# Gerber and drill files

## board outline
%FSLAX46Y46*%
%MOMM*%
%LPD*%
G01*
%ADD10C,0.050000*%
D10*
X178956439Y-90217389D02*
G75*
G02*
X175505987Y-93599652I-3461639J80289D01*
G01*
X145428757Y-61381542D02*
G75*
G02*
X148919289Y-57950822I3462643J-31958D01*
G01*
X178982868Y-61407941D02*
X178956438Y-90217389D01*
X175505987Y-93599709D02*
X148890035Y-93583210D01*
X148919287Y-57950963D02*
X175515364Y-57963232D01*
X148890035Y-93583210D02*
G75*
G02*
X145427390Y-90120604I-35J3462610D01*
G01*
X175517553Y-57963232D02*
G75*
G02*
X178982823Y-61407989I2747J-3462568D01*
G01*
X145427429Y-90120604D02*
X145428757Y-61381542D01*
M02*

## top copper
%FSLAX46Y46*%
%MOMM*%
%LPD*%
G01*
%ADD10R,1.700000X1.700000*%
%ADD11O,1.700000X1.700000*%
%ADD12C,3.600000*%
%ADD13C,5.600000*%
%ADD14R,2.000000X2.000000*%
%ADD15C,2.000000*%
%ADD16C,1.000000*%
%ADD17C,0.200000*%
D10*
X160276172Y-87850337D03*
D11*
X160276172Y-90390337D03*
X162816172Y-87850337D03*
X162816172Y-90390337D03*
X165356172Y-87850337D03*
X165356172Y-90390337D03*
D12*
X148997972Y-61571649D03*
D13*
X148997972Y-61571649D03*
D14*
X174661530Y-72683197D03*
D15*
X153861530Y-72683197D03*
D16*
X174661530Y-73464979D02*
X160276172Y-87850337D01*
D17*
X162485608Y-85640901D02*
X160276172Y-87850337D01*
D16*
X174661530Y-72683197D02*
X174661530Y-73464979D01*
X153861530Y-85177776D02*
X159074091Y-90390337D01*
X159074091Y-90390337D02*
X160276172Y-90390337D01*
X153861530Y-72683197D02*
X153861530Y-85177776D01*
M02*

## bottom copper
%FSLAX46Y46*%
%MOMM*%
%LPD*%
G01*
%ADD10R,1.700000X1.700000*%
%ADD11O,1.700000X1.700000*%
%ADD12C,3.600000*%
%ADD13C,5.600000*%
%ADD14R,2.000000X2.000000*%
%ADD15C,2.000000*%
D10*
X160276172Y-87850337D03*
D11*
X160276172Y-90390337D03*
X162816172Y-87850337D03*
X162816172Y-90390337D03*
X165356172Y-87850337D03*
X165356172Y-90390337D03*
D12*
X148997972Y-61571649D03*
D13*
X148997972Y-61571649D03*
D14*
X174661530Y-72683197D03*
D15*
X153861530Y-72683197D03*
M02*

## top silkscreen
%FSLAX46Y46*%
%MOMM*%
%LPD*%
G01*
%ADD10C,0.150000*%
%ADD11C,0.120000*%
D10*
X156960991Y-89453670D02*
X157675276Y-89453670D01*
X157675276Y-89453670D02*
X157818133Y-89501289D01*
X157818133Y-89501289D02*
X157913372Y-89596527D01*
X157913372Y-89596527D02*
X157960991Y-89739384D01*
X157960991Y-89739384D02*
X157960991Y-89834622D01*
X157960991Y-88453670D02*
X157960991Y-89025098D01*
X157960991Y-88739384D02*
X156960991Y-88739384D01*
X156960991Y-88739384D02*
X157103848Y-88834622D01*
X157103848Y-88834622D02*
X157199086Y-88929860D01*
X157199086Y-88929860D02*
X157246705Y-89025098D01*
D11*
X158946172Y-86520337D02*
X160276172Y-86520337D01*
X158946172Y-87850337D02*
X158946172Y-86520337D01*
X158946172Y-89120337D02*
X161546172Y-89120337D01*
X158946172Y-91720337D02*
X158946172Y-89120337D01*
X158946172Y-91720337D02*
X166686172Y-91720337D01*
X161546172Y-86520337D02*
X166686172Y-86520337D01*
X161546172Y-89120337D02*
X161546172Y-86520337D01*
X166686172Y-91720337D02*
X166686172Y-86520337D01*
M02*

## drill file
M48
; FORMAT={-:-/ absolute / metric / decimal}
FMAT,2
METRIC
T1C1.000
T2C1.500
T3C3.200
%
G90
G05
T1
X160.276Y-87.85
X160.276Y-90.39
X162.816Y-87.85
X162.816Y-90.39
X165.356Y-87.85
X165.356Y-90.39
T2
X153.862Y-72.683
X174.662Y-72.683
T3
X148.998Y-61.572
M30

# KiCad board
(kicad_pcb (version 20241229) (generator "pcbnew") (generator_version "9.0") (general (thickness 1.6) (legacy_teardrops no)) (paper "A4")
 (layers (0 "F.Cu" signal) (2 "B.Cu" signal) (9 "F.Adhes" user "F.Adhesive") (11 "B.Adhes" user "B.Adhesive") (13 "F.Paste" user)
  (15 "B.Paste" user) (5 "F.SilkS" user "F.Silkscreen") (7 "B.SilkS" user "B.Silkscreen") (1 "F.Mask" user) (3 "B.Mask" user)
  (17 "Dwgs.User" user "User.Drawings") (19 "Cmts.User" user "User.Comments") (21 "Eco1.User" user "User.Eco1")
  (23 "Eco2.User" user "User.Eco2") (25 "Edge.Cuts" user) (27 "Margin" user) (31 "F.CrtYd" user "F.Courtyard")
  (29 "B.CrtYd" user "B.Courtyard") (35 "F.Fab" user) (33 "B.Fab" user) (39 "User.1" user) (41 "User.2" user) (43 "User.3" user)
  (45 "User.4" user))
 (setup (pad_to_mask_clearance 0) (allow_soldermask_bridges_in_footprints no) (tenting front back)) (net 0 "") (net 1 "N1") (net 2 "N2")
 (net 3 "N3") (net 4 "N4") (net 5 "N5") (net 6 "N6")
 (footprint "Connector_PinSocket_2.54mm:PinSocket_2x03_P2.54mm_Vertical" (layer "F.Cu") (at 160.276172 87.850337 90)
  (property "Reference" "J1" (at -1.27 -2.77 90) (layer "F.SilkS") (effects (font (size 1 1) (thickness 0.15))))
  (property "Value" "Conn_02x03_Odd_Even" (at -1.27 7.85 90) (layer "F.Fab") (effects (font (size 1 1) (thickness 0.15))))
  (fp_line (start 1.33 -1.33) (end 1.33 0) (stroke (width 0.12) (type solid)) (layer "F.SilkS"))
  (fp_line (start 0 -1.33) (end 1.33 -1.33) (stroke (width 0.12) (type solid)) (layer "F.SilkS"))
  (fp_line (start -1.27 -1.33) (end -1.27 1.27) (stroke (width 0.12) (type solid)) (layer "F.SilkS"))
  (fp_line (start -3.87 -1.33) (end -1.27 -1.33) (stroke (width 0.12) (type solid)) (layer "F.SilkS"))
  (fp_line (start -3.87 -1.33) (end -3.87 6.41) (stroke (width 0.12) (type solid)) (layer "F.SilkS"))
  (fp_line (start 1.33 1.27) (end 1.33 6.41) (stroke (width 0.12) (type solid)) (layer "F.SilkS"))
  (fp_line (start -1.27 1.27) (end 1.33 1.27) (stroke (width 0.12) (type solid)) (layer "F.SilkS"))
  (fp_line (start -3.87 6.41) (end 1.33 6.41) (stroke (width 0.12) (type solid)) (layer "F.SilkS"))
  (pad "1" thru_hole rect (at 0 0 90) (size 1.7 1.7) (drill 1) (layers "*.Cu" "*.Mask") (remove_unused_layers no) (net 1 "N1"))
  (pad "2" thru_hole oval (at -2.54 0 90) (size 1.7 1.7) (drill 1) (layers "*.Cu" "*.Mask") (remove_unused_layers no) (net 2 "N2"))
  (pad "3" thru_hole oval (at 0 2.54 90) (size 1.7 1.7) (drill 1) (layers "*.Cu" "*.Mask") (remove_unused_layers no) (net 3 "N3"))
  (pad "4" thru_hole oval (at -2.54 2.54 90) (size 1.7 1.7) (drill 1) (layers "*.Cu" "*.Mask") (remove_unused_layers no) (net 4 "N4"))
  (pad "5" thru_hole oval (at 0 5.08 90) (size 1.7 1.7) (drill 1) (layers "*.Cu" "*.Mask") (remove_unused_layers no) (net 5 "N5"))
  (pad "6" thru_hole oval (at -2.54 5.08 90) (size 1.7 1.7) (drill 1) (layers "*.Cu" "*.Mask") (remove_unused_layers no) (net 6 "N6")))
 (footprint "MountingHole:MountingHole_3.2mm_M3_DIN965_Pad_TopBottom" (layer "F.Cu") (at 148.997972 61.571649)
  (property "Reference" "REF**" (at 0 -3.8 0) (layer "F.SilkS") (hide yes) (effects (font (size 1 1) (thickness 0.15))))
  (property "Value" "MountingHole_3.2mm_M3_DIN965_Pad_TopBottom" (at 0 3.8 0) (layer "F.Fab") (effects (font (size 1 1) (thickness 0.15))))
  (pad "1" thru_hole circle (at 0 0) (size 3.6 3.6) (drill 3.2) (layers "*.Cu" "*.Mask") (remove_unused_layers no))
  (pad "1" connect circle (at 0 0) (size 5.6 5.6) (layers "F.Cu" "F.Mask"))
  (pad "1" connect circle (at 0 0) (size 5.6 5.6) (layers "B.Cu" "B.Mask")))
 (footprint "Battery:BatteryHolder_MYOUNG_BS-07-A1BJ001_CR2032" (layer "B.Cu") (at 174.66153 72.683197 180)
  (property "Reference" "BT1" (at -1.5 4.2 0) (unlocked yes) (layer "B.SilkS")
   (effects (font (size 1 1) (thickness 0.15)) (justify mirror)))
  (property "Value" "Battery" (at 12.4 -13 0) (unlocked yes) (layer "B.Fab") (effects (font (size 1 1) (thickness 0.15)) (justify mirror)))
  (pad "1" thru_hole rect (at 0 0) (size 2 2) (drill 1.5) (layers "*.Cu" "*.Mask") (remove_unused_layers no) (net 1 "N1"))
  (pad "2" thru_hole circle (at 20.8 0) (size 2 2) (drill 1.5) (layers "*.Cu" "*.Mask") (remove_unused_layers no) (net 2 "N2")))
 (gr_arc (start 178.956439 90.217389) (mid 177.918661 92.609844) (end 175.505987 93.599709) (stroke (width 0.05) (type default))
  (layer "Edge.Cuts"))
 (gr_arc (start 145.428757 61.381542) (mid 146.464103 58.94391) (end 148.919288 57.950904) (stroke (width 0.05) (type default))
  (layer "Edge.Cuts"))
 (gr_line (start 178.982868 61.407941) (end 178.956438 90.217389) (stroke (width 0.05) (type default)) (layer "Edge.Cuts"))
 (gr_line (start 175.505987 93.599709) (end 148.890035 93.58321) (stroke (width 0.05) (type default)) (layer "Edge.Cuts"))
 (gr_line (start 148.919287 57.950963) (end 175.515364 57.963232) (stroke (width 0.05) (type default)) (layer "Edge.Cuts"))
 (gr_arc (start 148.890035 93.58321) (mid 146.441603 92.569036) (end 145.427429 90.120604) (stroke (width 0.05) (type default))
  (layer "Edge.Cuts"))
 (gr_arc (start 175.517553 57.963232) (mid 177.961445 58.970131) (end 178.982868 61.407989) (stroke (width 0.05) (type default))
  (layer "Edge.Cuts"))
 (gr_line (start 145.427429 90.120604) (end 145.428757 61.381542) (stroke (width 0.05) (type default)) (layer "Edge.Cuts"))
 (segment (start 174.66153 73.464979) (end 160.276172 87.850337) (width 1) (layer "F.Cu") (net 1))
 (segment (start 162.485608 85.640901) (end 160.276172 87.850337) (width 0.2) (layer "F.Cu") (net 1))
 (segment (start 174.66153 72.683197) (end 174.66153 73.464979) (width 1) (layer "F.Cu") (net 1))
 (segment (start 153.86153 85.177776) (end 159.074091 90.390337) (width 1) (layer "F.Cu") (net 2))
 (segment (start 159.074091 90.390337) (end 160.276172 90.390337) (width 1) (layer "F.Cu") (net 2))
 (segment (start 153.86153 72.683197) (end 153.86153 85.177776) (width 1) (layer "F.Cu") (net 2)))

